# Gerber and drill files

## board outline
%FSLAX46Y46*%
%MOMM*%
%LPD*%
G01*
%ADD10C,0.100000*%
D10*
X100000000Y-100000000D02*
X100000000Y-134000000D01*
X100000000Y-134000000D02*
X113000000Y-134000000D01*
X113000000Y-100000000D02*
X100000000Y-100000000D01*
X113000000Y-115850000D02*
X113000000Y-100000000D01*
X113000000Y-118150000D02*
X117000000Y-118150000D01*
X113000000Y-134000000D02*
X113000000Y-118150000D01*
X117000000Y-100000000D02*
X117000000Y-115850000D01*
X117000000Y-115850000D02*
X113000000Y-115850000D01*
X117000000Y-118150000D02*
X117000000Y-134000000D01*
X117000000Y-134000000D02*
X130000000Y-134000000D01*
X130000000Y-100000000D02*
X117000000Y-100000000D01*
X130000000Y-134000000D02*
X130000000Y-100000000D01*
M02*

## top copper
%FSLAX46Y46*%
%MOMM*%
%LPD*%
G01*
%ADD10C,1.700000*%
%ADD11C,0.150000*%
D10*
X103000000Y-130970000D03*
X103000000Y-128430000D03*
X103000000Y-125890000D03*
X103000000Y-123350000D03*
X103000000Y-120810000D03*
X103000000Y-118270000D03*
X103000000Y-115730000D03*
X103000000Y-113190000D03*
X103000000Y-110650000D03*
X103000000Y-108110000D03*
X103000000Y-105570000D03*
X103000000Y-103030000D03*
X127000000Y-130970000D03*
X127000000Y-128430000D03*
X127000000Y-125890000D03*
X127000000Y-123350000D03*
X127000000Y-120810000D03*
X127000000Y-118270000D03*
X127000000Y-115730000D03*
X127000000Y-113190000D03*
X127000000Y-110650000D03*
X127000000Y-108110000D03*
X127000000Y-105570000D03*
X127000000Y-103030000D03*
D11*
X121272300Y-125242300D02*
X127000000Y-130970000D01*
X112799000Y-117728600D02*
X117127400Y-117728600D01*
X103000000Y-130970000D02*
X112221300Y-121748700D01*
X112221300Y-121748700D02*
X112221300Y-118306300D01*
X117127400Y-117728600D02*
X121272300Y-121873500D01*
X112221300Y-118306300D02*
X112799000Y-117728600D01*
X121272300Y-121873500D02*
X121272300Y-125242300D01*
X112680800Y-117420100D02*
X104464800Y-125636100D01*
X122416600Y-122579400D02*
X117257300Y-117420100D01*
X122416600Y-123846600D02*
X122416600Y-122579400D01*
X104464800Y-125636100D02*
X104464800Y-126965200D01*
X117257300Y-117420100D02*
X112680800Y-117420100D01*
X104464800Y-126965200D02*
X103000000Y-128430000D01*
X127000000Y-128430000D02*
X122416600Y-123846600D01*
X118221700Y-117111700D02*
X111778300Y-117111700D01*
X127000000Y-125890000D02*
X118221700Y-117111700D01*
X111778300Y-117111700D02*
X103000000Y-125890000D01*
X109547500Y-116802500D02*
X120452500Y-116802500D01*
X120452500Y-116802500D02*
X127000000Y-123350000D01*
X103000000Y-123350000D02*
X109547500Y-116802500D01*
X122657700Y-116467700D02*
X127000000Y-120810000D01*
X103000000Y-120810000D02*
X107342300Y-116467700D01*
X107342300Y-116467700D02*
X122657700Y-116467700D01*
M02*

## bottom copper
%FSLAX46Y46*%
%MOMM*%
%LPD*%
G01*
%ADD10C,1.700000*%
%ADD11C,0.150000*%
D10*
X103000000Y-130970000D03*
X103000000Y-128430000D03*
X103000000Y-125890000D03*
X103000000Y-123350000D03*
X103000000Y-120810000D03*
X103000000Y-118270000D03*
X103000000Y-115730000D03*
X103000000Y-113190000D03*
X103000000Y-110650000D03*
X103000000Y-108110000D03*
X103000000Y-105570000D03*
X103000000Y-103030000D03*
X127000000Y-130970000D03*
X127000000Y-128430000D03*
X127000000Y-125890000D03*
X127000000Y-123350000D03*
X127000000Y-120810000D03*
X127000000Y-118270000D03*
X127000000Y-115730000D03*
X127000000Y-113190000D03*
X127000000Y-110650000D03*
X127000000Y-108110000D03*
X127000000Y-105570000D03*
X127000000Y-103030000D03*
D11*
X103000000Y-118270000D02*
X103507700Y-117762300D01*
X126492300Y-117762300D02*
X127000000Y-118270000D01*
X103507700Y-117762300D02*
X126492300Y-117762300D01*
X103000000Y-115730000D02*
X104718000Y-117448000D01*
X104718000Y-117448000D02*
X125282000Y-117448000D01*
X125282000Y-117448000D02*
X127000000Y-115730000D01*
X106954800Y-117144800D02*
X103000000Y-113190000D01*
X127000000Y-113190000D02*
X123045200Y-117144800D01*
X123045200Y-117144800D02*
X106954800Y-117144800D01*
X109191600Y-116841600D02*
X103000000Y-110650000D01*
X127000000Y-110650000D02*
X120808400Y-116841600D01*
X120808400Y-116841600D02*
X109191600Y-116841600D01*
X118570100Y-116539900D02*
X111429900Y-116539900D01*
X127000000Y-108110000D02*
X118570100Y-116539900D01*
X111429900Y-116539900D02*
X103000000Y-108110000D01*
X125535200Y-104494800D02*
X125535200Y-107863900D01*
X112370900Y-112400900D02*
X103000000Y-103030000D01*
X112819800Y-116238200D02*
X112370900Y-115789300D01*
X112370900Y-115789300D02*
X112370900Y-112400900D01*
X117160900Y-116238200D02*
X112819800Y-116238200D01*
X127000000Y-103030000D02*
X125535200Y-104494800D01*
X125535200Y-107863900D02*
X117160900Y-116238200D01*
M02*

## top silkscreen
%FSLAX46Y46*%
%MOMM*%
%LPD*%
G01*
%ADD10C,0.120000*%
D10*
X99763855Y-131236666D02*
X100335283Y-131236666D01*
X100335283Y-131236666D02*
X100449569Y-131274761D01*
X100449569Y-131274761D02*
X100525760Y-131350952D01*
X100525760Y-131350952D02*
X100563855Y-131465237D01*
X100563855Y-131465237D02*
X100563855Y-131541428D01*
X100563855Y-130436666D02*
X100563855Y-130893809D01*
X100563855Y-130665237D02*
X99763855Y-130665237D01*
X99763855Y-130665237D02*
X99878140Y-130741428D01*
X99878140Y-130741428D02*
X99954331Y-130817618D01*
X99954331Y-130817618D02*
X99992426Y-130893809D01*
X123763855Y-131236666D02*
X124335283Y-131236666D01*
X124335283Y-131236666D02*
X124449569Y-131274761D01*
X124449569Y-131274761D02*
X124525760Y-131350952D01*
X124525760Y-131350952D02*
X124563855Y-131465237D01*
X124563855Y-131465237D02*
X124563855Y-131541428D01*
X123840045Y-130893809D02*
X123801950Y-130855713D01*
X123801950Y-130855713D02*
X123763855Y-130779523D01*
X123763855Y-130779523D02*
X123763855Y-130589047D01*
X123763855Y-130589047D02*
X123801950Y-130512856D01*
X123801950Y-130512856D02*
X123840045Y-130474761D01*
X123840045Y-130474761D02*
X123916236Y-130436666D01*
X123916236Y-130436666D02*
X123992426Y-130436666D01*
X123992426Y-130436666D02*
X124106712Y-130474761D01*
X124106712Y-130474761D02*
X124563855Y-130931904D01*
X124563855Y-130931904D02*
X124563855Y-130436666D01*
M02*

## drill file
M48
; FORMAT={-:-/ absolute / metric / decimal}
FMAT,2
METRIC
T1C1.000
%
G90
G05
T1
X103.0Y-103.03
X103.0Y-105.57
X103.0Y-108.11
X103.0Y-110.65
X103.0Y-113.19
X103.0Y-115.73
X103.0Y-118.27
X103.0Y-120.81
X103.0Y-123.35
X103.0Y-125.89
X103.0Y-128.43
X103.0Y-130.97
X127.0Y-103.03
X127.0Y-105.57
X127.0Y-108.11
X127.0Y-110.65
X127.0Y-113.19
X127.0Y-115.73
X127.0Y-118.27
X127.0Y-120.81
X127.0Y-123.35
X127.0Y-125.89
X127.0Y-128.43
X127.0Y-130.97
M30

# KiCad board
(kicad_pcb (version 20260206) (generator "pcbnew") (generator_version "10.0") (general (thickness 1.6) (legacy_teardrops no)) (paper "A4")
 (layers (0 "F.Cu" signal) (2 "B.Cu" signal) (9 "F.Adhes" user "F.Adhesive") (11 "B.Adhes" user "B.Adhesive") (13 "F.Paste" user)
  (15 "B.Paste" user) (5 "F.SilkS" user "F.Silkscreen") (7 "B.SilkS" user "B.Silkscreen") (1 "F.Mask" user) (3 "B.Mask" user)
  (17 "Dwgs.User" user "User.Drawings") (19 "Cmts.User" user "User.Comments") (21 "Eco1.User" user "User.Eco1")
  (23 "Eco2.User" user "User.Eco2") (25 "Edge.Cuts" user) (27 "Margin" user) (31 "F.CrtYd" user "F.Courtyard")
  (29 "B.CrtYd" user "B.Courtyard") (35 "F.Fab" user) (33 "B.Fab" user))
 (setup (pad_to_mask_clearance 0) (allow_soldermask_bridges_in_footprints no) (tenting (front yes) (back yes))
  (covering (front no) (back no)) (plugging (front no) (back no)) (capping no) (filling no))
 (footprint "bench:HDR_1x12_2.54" (layer "F.Cu") (at 103 130.97 90)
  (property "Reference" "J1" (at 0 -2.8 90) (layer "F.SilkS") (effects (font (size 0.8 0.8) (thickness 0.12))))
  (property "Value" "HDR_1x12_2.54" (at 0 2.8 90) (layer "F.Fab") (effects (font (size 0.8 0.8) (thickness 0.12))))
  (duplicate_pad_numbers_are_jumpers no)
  (pad "1" thru_hole circle (at 0 0 90) (size 1.7 1.7) (drill 1) (layers "*.Cu" "*.Mask") (remove_unused_layers no) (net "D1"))
  (pad "2" thru_hole circle (at 2.54 0 90) (size 1.7 1.7) (drill 1) (layers "*.Cu" "*.Mask") (remove_unused_layers no) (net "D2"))
  (pad "3" thru_hole circle (at 5.08 0 90) (size 1.7 1.7) (drill 1) (layers "*.Cu" "*.Mask") (remove_unused_layers no) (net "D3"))
  (pad "4" thru_hole circle (at 7.62 0 90) (size 1.7 1.7) (drill 1) (layers "*.Cu" "*.Mask") (remove_unused_layers no) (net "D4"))
  (pad "5" thru_hole circle (at 10.16 0 90) (size 1.7 1.7) (drill 1) (layers "*.Cu" "*.Mask") (remove_unused_layers no) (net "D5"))
  (pad "6" thru_hole circle (at 12.7 0 90) (size 1.7 1.7) (drill 1) (layers "*.Cu" "*.Mask") (remove_unused_layers no) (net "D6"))
  (pad "7" thru_hole circle (at 15.24 0 90) (size 1.7 1.7) (drill 1) (layers "*.Cu" "*.Mask") (remove_unused_layers no) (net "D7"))
  (pad "8" thru_hole circle (at 17.78 0 90) (size 1.7 1.7) (drill 1) (layers "*.Cu" "*.Mask") (remove_unused_layers no) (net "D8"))
  (pad "9" thru_hole circle (at 20.32 0 90) (size 1.7 1.7) (drill 1) (layers "*.Cu" "*.Mask") (remove_unused_layers no) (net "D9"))
  (pad "10" thru_hole circle (at 22.86 0 90) (size 1.7 1.7) (drill 1) (layers "*.Cu" "*.Mask") (remove_unused_layers no) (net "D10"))
  (pad "11" thru_hole circle (at 25.4 0 90) (size 1.7 1.7) (drill 1) (layers "*.Cu" "*.Mask") (remove_unused_layers no) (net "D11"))
  (pad "12" thru_hole circle (at 27.94 0 90) (size 1.7 1.7) (drill 1) (layers "*.Cu" "*.Mask") (remove_unused_layers no) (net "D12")))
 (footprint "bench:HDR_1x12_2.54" (layer "F.Cu") (at 127 130.97 90)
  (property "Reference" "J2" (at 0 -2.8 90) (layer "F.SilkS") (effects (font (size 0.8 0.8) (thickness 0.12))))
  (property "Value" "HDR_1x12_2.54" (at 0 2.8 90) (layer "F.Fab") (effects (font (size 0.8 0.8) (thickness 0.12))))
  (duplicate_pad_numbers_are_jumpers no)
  (pad "1" thru_hole circle (at 0 0 90) (size 1.7 1.7) (drill 1) (layers "*.Cu" "*.Mask") (remove_unused_layers no) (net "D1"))
  (pad "2" thru_hole circle (at 2.54 0 90) (size 1.7 1.7) (drill 1) (layers "*.Cu" "*.Mask") (remove_unused_layers no) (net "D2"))
  (pad "3" thru_hole circle (at 5.08 0 90) (size 1.7 1.7) (drill 1) (layers "*.Cu" "*.Mask") (remove_unused_layers no) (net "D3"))
  (pad "4" thru_hole circle (at 7.62 0 90) (size 1.7 1.7) (drill 1) (layers "*.Cu" "*.Mask") (remove_unused_layers no) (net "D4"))
  (pad "5" thru_hole circle (at 10.16 0 90) (size 1.7 1.7) (drill 1) (layers "*.Cu" "*.Mask") (remove_unused_layers no) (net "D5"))
  (pad "6" thru_hole circle (at 12.7 0 90) (size 1.7 1.7) (drill 1) (layers "*.Cu" "*.Mask") (remove_unused_layers no) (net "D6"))
  (pad "7" thru_hole circle (at 15.24 0 90) (size 1.7 1.7) (drill 1) (layers "*.Cu" "*.Mask") (remove_unused_layers no) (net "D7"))
  (pad "8" thru_hole circle (at 17.78 0 90) (size 1.7 1.7) (drill 1) (layers "*.Cu" "*.Mask") (remove_unused_layers no) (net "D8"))
  (pad "9" thru_hole circle (at 20.32 0 90) (size 1.7 1.7) (drill 1) (layers "*.Cu" "*.Mask") (remove_unused_layers no) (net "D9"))
  (pad "10" thru_hole circle (at 22.86 0 90) (size 1.7 1.7) (drill 1) (layers "*.Cu" "*.Mask") (remove_unused_layers no) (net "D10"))
  (pad "11" thru_hole circle (at 25.4 0 90) (size 1.7 1.7) (drill 1) (layers "*.Cu" "*.Mask") (remove_unused_layers no) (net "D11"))
  (pad "12" thru_hole circle (at 27.94 0 90) (size 1.7 1.7) (drill 1) (layers "*.Cu" "*.Mask") (remove_unused_layers no) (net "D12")))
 (gr_line (start 100 100) (end 100 134) (stroke (width 0.1) (type solid)) (layer "Edge.Cuts"))
 (gr_line (start 100 134) (end 113 134) (stroke (width 0.1) (type solid)) (layer "Edge.Cuts"))
 (gr_line (start 113 100) (end 100 100) (stroke (width 0.1) (type solid)) (layer "Edge.Cuts"))
 (gr_line (start 113 115.85) (end 113 100) (stroke (width 0.1) (type solid)) (layer "Edge.Cuts"))
 (gr_line (start 113 118.15) (end 117 118.15) (stroke (width 0.1) (type solid)) (layer "Edge.Cuts"))
 (gr_line (start 113 134) (end 113 118.15) (stroke (width 0.1) (type solid)) (layer "Edge.Cuts"))
 (gr_line (start 117 100) (end 117 115.85) (stroke (width 0.1) (type solid)) (layer "Edge.Cuts"))
 (gr_line (start 117 115.85) (end 113 115.85) (stroke (width 0.1) (type solid)) (layer "Edge.Cuts"))
 (gr_line (start 117 118.15) (end 117 134) (stroke (width 0.1) (type solid)) (layer "Edge.Cuts"))
 (gr_line (start 117 134) (end 130 134) (stroke (width 0.1) (type solid)) (layer "Edge.Cuts"))
 (gr_line (start 130 100) (end 117 100) (stroke (width 0.1) (type solid)) (layer "Edge.Cuts"))
 (gr_line (start 130 134) (end 130 100) (stroke (width 0.1) (type solid)) (layer "Edge.Cuts"))
 (segment (start 121.2723 125.2423) (end 127 130.97) (width 0.15) (layer "F.Cu") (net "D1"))
 (segment (start 112.799 117.7286) (end 117.1274 117.7286) (width 0.15) (layer "F.Cu") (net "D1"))
 (segment (start 103 130.97) (end 112.2213 121.7487) (width 0.15) (layer "F.Cu") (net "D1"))
 (segment (start 112.2213 121.7487) (end 112.2213 118.3063) (width 0.15) (layer "F.Cu") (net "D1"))
 (segment (start 117.1274 117.7286) (end 121.2723 121.8735) (width 0.15) (layer "F.Cu") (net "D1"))
 (segment (start 112.2213 118.3063) (end 112.799 117.7286) (width 0.15) (layer "F.Cu") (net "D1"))
 (segment (start 121.2723 121.8735) (end 121.2723 125.2423) (width 0.15) (layer "F.Cu") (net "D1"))
 (segment (start 112.6808 117.4201) (end 104.4648 125.6361) (width 0.15) (layer "F.Cu") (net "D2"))
 (segment (start 122.4166 122.5794) (end 117.2573 117.4201) (width 0.15) (layer "F.Cu") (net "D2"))
 (segment (start 122.4166 123.8466) (end 122.4166 122.5794) (width 0.15) (layer "F.Cu") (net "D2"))
 (segment (start 104.4648 125.6361) (end 104.4648 126.9652) (width 0.15) (layer "F.Cu") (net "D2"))
 (segment (start 117.2573 117.4201) (end 112.6808 117.4201) (width 0.15) (layer "F.Cu") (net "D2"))
 (segment (start 104.4648 126.9652) (end 103 128.43) (width 0.15) (layer "F.Cu") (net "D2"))
 (segment (start 127 128.43) (end 122.4166 123.8466) (width 0.15) (layer "F.Cu") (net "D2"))
 (segment (start 118.2217 117.1117) (end 111.7783 117.1117) (width 0.15) (layer "F.Cu") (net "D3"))
 (segment (start 127 125.89) (end 118.2217 117.1117) (width 0.15) (layer "F.Cu") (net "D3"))
 (segment (start 111.7783 117.1117) (end 103 125.89) (width 0.15) (layer "F.Cu") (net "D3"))
 (segment (start 109.5475 116.8025) (end 120.4525 116.8025) (width 0.15) (layer "F.Cu") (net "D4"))
 (segment (start 120.4525 116.8025) (end 127 123.35) (width 0.15) (layer "F.Cu") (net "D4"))
 (segment (start 103 123.35) (end 109.5475 116.8025) (width 0.15) (layer "F.Cu") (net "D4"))
 (segment (start 122.6577 116.4677) (end 127 120.81) (width 0.15) (layer "F.Cu") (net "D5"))
 (segment (start 103 120.81) (end 107.3423 116.4677) (width 0.15) (layer "F.Cu") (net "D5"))
 (segment (start 107.3423 116.4677) (end 122.6577 116.4677) (width 0.15) (layer "F.Cu") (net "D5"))
 (segment (start 103 118.27) (end 103.5077 117.7623) (width 0.15) (layer "B.Cu") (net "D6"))
 (segment (start 126.4923 117.7623) (end 127 118.27) (width 0.15) (layer "B.Cu") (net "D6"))
 (segment (start 103.5077 117.7623) (end 126.4923 117.7623) (width 0.15) (layer "B.Cu") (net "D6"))
 (segment (start 103 115.73) (end 104.718 117.448) (width 0.15) (layer "B.Cu") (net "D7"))
 (segment (start 104.718 117.448) (end 125.282 117.448) (width 0.15) (layer "B.Cu") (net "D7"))
 (segment (start 125.282 117.448) (end 127 115.73) (width 0.15) (layer "B.Cu") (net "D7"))
 (segment (start 106.9548 117.1448) (end 103 113.19) (width 0.15) (layer "B.Cu") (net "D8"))
 (segment (start 127 113.19) (end 123.0452 117.1448) (width 0.15) (layer "B.Cu") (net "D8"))
 (segment (start 123.0452 117.1448) (end 106.9548 117.1448) (width 0.15) (layer "B.Cu") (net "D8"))
 (segment (start 109.1916 116.8416) (end 103 110.65) (width 0.15) (layer "B.Cu") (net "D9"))
 (segment (start 127 110.65) (end 120.8084 116.8416) (width 0.15) (layer "B.Cu") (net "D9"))
 (segment (start 120.8084 116.8416) (end 109.1916 116.8416) (width 0.15) (layer "B.Cu") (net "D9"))
 (segment (start 118.5701 116.5399) (end 111.4299 116.5399) (width 0.15) (layer "B.Cu") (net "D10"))
 (segment (start 127 108.11) (end 118.5701 116.5399) (width 0.15) (layer "B.Cu") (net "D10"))
 (segment (start 111.4299 116.5399) (end 103 108.11) (width 0.15) (layer "B.Cu") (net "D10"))
 (segment (start 125.5352 104.4948) (end 125.5352 107.8639) (width 0.15) (layer "B.Cu") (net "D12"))
 (segment (start 112.3709 112.4009) (end 103 103.03) (width 0.15) (layer "B.Cu") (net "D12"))
 (segment (start 112.8198 116.2382) (end 112.3709 115.7893) (width 0.15) (layer "B.Cu") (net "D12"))
 (segment (start 112.3709 115.7893) (end 112.3709 112.4009) (width 0.15) (layer "B.Cu") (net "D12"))
 (segment (start 117.1609 116.2382) (end 112.8198 116.2382) (width 0.15) (layer "B.Cu") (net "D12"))
 (segment (start 127 103.03) (end 125.5352 104.4948) (width 0.15) (layer "B.Cu") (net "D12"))
 (segment (start 125.5352 107.8639) (end 117.1609 116.2382) (width 0.15) (layer "B.Cu") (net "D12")))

